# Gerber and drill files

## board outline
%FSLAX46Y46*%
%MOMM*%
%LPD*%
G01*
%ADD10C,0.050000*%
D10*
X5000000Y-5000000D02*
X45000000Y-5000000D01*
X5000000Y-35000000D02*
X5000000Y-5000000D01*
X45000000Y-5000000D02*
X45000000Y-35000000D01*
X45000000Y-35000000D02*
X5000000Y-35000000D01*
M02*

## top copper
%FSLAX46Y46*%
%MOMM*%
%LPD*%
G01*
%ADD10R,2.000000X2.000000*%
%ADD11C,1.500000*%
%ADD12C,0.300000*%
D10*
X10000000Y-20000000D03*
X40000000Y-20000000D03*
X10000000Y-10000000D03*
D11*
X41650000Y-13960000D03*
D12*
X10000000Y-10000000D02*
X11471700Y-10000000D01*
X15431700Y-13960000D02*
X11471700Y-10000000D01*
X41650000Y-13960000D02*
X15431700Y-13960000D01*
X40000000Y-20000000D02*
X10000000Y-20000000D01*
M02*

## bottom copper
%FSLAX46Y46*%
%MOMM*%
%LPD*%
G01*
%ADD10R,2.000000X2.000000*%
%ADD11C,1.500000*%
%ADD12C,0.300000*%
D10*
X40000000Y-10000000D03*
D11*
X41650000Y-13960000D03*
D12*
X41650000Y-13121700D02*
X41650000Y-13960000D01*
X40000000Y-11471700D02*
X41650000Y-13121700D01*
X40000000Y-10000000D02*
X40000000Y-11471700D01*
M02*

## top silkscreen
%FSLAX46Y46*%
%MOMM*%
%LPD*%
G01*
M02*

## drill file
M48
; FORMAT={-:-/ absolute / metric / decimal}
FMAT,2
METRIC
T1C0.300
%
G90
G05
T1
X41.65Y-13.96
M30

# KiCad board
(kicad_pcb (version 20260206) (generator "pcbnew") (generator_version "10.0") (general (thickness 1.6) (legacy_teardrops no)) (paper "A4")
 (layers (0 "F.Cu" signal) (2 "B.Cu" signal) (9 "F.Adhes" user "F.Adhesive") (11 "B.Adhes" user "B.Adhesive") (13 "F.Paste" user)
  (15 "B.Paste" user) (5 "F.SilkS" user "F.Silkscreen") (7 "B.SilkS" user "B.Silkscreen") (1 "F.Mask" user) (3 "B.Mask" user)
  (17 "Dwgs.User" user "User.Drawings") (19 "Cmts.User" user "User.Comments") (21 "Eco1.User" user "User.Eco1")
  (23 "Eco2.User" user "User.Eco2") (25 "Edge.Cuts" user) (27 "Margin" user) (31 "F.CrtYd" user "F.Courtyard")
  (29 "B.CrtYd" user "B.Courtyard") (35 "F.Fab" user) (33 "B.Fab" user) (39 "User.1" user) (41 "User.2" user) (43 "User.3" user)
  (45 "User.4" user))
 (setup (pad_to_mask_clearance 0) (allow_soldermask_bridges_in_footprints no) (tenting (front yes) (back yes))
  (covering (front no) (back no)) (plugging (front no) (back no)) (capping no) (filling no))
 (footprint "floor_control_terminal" (layer "F.Cu") (at 10 20)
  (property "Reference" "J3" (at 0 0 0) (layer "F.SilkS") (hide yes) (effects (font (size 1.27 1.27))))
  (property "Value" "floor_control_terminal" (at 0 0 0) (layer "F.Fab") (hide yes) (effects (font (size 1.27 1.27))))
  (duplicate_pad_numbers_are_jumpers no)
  (pad "1" smd rect (at 0 0) (size 2 2) (layers "F.Cu" "F.Mask" "F.Paste") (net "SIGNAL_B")))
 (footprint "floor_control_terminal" (layer "F.Cu") (at 40 20)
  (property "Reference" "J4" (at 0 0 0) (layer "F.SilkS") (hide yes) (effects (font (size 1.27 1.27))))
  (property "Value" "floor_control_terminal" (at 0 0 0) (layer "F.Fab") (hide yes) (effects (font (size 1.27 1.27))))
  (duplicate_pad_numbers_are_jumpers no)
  (pad "1" smd rect (at 0 0) (size 2 2) (layers "F.Cu" "F.Mask" "F.Paste") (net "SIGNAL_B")))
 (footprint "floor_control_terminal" (layer "F.Cu") (at 10 10)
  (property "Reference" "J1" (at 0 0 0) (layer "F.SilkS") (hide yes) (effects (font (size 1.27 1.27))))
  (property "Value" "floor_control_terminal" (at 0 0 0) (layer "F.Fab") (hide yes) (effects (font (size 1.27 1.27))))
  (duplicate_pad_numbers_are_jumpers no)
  (pad "1" smd rect (at 0 0) (size 2 2) (layers "F.Cu" "F.Mask" "F.Paste") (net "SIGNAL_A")))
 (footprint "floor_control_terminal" (layer "B.Cu") (at 40 10)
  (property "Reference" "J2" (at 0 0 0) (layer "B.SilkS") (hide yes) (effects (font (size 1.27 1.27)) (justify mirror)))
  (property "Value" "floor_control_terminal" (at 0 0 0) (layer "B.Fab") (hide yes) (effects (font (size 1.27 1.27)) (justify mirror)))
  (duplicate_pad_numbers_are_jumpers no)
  (pad "1" smd rect (at 0 0) (size 2 2) (layers "B.Cu" "B.Mask" "B.Paste") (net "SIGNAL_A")))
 (gr_line (start 5 5) (end 45 5) (stroke (width 0.05) (type default)) (layer "Edge.Cuts"))
 (gr_line (start 5 35) (end 5 5) (stroke (width 0.05) (type default)) (layer "Edge.Cuts"))
 (gr_line (start 45 5) (end 45 35) (stroke (width 0.05) (type default)) (layer "Edge.Cuts"))
 (gr_line (start 45 35) (end 5 35) (stroke (width 0.05) (type default)) (layer "Edge.Cuts"))
 (segment (start 10 10) (end 11.4717 10) (width 0.3) (layer "F.Cu") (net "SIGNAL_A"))
 (segment (start 15.4317 13.96) (end 11.4717 10) (width 0.3) (layer "F.Cu") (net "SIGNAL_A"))
 (segment (start 41.65 13.96) (end 15.4317 13.96) (width 0.3) (layer "F.Cu") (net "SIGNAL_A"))
 (via (at 41.65 13.96) (size 1.5) (drill 0.3) (layers "F.Cu" "B.Cu") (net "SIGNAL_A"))
 (segment (start 41.65 13.1217) (end 41.65 13.96) (width 0.3) (layer "B.Cu") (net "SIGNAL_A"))
 (segment (start 40 11.4717) (end 41.65 13.1217) (width 0.3) (layer "B.Cu") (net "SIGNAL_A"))
 (segment (start 40 10) (end 40 11.4717) (width 0.3) (layer "B.Cu") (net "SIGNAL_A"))
 (segment (start 40 20) (end 10 20) (width 0.3) (layer "F.Cu") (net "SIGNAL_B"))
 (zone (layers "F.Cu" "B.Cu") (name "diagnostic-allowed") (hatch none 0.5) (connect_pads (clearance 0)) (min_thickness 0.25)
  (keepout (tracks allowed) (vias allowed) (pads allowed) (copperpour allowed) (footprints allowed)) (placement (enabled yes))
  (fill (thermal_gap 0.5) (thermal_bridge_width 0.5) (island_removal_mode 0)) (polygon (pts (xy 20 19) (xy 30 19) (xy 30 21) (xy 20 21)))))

